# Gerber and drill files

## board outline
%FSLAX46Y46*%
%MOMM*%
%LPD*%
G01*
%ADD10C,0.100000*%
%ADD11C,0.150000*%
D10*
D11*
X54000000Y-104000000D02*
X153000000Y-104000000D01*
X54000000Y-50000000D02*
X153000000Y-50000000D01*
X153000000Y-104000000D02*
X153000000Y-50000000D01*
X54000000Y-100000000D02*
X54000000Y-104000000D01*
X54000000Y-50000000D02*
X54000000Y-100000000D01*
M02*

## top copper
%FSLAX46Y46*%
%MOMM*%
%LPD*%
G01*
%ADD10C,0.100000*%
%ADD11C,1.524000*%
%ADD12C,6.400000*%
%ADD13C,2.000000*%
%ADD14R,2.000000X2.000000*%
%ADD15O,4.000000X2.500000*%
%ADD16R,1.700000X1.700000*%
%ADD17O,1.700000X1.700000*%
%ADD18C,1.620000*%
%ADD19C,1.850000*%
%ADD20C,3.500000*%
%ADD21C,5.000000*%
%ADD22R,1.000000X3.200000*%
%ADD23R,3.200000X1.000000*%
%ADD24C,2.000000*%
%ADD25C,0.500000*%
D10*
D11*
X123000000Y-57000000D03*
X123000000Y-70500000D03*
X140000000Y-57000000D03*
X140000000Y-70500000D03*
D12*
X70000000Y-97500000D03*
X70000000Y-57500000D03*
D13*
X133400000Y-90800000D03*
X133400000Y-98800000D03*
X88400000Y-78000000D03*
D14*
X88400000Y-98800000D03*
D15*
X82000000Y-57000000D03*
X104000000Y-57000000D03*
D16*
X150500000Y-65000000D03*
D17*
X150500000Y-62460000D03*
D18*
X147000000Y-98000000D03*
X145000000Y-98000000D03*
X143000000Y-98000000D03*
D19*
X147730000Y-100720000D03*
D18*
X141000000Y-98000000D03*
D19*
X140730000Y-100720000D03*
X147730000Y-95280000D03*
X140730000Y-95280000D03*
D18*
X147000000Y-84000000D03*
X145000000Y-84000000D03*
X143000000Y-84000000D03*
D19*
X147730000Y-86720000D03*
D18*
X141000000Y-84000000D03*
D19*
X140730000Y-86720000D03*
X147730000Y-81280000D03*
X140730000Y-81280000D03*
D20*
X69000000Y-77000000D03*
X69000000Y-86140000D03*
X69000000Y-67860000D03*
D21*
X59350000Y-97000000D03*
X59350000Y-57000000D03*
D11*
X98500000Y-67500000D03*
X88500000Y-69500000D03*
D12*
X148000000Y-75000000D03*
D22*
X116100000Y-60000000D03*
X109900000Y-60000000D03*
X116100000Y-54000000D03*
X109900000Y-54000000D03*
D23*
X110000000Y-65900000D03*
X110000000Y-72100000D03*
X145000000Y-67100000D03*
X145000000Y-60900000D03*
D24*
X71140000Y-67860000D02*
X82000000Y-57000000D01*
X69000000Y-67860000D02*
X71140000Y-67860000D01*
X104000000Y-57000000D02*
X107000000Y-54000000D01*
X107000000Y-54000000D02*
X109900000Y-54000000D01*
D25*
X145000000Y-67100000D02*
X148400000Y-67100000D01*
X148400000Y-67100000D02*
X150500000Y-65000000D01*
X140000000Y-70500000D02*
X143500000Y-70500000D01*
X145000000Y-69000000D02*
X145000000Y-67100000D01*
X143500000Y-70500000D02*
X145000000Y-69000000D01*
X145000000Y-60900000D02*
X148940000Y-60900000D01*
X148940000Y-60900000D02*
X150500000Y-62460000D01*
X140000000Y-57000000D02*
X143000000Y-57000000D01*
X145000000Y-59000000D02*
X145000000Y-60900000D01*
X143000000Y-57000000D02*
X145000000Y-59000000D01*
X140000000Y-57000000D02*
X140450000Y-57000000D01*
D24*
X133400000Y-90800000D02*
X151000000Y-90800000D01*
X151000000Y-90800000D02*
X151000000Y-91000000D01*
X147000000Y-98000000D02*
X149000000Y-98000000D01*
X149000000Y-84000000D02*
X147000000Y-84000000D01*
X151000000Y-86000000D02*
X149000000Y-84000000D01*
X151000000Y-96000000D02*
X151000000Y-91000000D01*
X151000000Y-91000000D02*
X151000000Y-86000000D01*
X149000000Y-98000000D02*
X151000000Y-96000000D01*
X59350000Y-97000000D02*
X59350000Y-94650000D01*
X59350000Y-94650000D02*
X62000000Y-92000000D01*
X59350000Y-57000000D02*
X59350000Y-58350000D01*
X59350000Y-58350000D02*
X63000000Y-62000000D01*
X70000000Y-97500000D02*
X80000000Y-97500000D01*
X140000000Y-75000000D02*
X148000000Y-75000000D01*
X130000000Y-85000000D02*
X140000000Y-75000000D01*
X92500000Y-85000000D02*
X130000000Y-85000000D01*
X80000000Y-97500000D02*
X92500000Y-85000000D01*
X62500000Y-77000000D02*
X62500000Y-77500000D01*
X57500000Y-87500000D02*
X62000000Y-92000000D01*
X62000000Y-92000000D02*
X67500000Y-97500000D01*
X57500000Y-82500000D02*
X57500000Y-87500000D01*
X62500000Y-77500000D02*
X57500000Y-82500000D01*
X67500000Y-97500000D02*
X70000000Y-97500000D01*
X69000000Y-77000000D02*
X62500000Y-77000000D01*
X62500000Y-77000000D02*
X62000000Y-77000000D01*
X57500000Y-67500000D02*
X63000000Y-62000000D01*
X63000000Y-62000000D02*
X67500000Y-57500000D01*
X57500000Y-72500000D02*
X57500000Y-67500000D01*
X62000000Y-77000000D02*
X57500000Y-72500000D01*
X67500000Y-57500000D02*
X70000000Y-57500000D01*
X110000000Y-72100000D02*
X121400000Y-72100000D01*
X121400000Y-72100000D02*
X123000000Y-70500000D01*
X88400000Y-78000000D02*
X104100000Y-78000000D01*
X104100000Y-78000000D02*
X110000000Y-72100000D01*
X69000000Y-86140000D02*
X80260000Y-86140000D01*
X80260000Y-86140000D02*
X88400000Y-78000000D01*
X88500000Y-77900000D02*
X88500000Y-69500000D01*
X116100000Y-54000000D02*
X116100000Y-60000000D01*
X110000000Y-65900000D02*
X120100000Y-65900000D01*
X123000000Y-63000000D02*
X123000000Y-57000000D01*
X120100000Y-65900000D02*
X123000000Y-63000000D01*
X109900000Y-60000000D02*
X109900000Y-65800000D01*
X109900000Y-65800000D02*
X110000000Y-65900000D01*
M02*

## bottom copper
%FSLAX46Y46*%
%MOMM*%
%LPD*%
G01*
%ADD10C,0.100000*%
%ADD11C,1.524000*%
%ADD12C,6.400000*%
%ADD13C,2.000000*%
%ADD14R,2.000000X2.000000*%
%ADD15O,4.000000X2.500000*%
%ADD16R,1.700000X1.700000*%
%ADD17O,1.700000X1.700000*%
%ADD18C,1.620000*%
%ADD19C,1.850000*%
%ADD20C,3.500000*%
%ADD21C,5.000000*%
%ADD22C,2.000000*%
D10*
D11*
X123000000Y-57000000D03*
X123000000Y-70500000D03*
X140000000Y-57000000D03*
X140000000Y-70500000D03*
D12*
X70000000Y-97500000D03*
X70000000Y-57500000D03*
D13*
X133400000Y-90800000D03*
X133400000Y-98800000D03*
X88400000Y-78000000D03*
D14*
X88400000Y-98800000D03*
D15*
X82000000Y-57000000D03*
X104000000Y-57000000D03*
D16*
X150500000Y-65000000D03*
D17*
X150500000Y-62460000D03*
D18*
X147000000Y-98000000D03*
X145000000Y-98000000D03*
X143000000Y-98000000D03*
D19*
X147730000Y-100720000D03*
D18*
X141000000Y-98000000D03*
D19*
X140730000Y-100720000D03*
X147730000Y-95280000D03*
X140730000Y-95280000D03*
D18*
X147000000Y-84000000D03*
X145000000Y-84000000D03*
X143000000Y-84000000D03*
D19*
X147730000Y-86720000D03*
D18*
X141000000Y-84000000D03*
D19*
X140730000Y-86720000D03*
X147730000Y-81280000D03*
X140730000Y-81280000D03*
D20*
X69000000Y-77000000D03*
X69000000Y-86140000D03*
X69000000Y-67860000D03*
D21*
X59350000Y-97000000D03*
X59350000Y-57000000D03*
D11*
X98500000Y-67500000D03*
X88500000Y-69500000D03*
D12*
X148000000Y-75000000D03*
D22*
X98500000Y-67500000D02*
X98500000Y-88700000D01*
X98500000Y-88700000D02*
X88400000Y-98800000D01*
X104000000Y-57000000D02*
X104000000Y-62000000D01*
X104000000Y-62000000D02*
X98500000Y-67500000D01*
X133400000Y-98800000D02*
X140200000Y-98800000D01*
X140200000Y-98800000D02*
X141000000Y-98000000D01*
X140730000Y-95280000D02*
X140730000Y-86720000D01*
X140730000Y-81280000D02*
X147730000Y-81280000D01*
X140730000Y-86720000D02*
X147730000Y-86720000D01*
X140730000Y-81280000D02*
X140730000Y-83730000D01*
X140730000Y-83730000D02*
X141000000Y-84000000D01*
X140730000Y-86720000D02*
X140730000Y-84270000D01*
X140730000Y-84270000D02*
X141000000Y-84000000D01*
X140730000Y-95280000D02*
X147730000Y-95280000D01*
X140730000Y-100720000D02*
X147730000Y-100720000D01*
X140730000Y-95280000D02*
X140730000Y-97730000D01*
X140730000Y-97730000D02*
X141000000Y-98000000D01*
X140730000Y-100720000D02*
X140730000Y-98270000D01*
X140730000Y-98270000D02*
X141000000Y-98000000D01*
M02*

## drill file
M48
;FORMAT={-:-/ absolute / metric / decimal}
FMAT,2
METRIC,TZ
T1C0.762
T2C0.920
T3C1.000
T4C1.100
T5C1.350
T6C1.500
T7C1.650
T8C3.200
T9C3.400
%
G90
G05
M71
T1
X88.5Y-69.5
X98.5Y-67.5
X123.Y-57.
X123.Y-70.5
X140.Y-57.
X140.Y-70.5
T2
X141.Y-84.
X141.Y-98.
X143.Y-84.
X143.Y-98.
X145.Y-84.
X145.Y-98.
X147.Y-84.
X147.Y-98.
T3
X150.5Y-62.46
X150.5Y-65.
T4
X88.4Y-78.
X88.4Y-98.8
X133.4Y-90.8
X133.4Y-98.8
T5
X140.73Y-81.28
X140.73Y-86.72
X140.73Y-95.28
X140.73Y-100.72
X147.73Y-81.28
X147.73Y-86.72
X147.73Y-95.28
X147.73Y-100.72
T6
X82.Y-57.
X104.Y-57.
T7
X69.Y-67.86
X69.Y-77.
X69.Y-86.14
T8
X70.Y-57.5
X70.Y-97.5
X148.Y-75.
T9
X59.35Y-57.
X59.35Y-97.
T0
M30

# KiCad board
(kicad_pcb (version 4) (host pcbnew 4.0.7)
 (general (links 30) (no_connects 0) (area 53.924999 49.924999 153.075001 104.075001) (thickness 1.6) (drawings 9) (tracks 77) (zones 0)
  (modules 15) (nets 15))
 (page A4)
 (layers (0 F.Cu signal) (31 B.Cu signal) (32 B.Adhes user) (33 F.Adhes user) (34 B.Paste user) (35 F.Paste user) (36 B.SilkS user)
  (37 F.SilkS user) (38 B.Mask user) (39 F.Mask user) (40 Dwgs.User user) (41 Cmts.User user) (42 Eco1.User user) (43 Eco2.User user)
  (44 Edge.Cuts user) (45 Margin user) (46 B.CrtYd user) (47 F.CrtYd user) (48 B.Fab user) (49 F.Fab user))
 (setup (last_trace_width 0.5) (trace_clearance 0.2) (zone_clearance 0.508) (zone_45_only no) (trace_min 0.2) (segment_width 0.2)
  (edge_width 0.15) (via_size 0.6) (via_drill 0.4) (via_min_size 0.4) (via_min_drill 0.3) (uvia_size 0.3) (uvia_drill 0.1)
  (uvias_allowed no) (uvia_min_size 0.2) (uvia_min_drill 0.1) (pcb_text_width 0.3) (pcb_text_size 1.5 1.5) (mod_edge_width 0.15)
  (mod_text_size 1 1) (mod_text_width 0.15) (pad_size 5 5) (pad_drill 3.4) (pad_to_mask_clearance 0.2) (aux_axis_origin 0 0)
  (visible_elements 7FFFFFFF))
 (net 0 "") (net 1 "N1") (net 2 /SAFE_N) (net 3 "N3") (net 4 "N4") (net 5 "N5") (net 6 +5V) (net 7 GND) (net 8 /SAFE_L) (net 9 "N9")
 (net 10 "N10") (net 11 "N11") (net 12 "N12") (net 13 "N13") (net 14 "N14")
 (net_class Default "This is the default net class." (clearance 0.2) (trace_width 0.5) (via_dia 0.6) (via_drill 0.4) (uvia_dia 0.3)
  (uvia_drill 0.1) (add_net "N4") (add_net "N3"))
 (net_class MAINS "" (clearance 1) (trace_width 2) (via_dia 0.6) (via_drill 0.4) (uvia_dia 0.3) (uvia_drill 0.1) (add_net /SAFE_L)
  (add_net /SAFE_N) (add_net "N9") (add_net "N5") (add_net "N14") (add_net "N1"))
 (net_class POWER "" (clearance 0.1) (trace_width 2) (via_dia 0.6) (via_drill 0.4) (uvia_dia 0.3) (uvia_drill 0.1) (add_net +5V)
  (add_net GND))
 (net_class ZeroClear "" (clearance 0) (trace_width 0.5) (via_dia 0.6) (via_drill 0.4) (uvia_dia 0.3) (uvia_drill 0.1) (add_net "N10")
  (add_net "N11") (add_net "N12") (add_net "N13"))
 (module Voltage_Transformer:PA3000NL (layer F.Cu) (at 123 57)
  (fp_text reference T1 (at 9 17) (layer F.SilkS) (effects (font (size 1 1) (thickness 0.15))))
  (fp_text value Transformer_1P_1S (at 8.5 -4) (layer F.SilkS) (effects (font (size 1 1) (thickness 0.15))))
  (pad 1 thru_hole circle (at 0 0) (size 1.524 1.524) (drill 0.762) (layers *.Cu *.Mask) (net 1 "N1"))
  (pad 2 thru_hole circle (at 0 13.5) (size 1.524 1.524) (drill 0.762) (layers *.Cu *.Mask) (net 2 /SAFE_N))
  (pad 3 thru_hole circle (at 17 0) (size 1.524 1.524) (drill 0.762) (layers *.Cu *.Mask) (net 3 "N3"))
  (pad 4 thru_hole circle (at 17 13.5) (size 1.524 1.524) (drill 0.762) (layers *.Cu *.Mask) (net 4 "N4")))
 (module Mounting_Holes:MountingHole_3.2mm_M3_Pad (layer F.Cu) (at 70 97.5)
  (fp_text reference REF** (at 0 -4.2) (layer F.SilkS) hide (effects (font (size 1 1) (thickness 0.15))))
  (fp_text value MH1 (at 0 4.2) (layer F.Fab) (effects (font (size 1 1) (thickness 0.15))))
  (pad 1 thru_hole circle (at 0 0) (size 6.4 6.4) (drill 3.2) (layers *.Cu *.Mask) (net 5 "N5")))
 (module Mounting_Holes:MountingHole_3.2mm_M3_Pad (layer F.Cu) (at 70 57.5)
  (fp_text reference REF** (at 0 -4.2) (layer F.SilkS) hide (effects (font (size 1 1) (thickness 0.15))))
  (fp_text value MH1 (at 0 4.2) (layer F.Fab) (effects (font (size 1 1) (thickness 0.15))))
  (pad 1 thru_hole circle (at 0 0) (size 6.4 6.4) (drill 3.2) (layers *.Cu *.Mask) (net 5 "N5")))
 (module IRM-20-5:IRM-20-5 (layer F.Cu) (at 85 102)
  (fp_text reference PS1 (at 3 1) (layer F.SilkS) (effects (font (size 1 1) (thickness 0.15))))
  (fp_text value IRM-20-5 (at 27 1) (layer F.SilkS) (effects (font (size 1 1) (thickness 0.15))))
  (pad 4 thru_hole circle (at 48.4 -11.2 270) (size 2 2) (drill 1.1) (layers *.Cu *.Mask) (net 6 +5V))
  (pad 3 thru_hole circle (at 48.4 -3.2 270) (size 2 2) (drill 1.1) (layers *.Cu *.Mask) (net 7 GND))
  (pad 2 thru_hole circle (at 3.4 -24 270) (size 2 2) (drill 1.1) (layers *.Cu *.Mask) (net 2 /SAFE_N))
  (pad 1 thru_hole rect (at 3.4 -3.2 270) (size 2 2) (drill 1.1) (layers *.Cu *.Mask) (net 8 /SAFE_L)))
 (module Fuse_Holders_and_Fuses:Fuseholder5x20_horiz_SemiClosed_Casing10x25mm (layer F.Cu) (at 104 57 180)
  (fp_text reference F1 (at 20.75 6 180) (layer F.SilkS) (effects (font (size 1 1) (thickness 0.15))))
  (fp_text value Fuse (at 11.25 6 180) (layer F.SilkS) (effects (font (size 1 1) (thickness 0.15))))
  (pad 2 thru_hole oval (at 22 0 90) (size 2.5 4) (drill 1.5) (layers *.Cu *.Mask) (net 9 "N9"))
  (pad 1 thru_hole oval (at 0 0 90) (size 2.5 4) (drill 1.5) (layers *.Cu *.Mask) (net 8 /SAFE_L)))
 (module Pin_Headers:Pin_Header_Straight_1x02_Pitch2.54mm (layer F.Cu) (at 150.5 65 180)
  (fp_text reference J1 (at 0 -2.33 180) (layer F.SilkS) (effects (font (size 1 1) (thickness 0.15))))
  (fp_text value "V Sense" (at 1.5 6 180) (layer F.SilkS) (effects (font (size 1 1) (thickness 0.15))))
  (pad 1 thru_hole rect (at 0 0 180) (size 1.7 1.7) (drill 1) (layers *.Cu *.Mask) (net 4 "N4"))
  (pad 2 thru_hole oval (at 0 2.54 180) (size 1.7 1.7) (drill 1) (layers *.Cu *.Mask) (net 3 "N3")))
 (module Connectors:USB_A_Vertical (layer F.Cu) (at 147 98 270)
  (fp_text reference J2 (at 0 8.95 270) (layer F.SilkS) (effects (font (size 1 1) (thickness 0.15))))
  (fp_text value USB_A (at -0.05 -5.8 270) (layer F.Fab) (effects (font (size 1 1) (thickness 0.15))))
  (pad 1 thru_hole circle (at 0 0 270) (size 1.62 1.62) (drill 0.92) (layers *.Cu *.Mask) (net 6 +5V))
  (pad 2 thru_hole circle (at 0 2 270) (size 1.62 1.62) (drill 0.92) (layers *.Cu *.Mask) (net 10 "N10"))
  (pad 3 thru_hole circle (at 0 4 270) (size 1.62 1.62) (drill 0.92) (layers *.Cu *.Mask) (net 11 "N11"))
  (pad 5 thru_hole circle (at 2.72 -0.73 270) (size 1.85 1.85) (drill 1.35) (layers *.Cu *.Mask) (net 7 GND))
  (pad 4 thru_hole circle (at 0 6 270) (size 1.62 1.62) (drill 0.92) (layers *.Cu *.Mask) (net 7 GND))
  (pad 5 thru_hole circle (at 2.72 6.27 270) (size 1.85 1.85) (drill 1.35) (layers *.Cu *.Mask) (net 7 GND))
  (pad 5 thru_hole circle (at -2.72 -0.73 270) (size 1.85 1.85) (drill 1.35) (layers *.Cu *.Mask) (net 7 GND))
  (pad 5 thru_hole circle (at -2.72 6.27 270) (size 1.85 1.85) (drill 1.35) (layers *.Cu *.Mask) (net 7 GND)))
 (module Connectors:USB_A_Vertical (layer F.Cu) (at 147 84 270)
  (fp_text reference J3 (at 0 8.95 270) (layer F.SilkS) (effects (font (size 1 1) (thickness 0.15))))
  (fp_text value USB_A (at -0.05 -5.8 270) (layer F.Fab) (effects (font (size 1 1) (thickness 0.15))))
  (pad 1 thru_hole circle (at 0 0 270) (size 1.62 1.62) (drill 0.92) (layers *.Cu *.Mask) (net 6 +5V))
  (pad 2 thru_hole circle (at 0 2 270) (size 1.62 1.62) (drill 0.92) (layers *.Cu *.Mask) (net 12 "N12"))
  (pad 3 thru_hole circle (at 0 4 270) (size 1.62 1.62) (drill 0.92) (layers *.Cu *.Mask) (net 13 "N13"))
  (pad 5 thru_hole circle (at 2.72 -0.73 270) (size 1.85 1.85) (drill 1.35) (layers *.Cu *.Mask) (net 7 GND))
  (pad 4 thru_hole circle (at 0 6 270) (size 1.62 1.62) (drill 0.92) (layers *.Cu *.Mask) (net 7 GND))
  (pad 5 thru_hole circle (at 2.72 6.27 270) (size 1.85 1.85) (drill 1.35) (layers *.Cu *.Mask) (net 7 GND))
  (pad 5 thru_hole circle (at -2.72 -0.73 270) (size 1.85 1.85) (drill 1.35) (layers *.Cu *.Mask) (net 7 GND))
  (pad 5 thru_hole circle (at -2.72 6.27 270) (size 1.85 1.85) (drill 1.35) (layers *.Cu *.Mask) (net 7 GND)))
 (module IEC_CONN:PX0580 (layer F.Cu) (at 69 77 90)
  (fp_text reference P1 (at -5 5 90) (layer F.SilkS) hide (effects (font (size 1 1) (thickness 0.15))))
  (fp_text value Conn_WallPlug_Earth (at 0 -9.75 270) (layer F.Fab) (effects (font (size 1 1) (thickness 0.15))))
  (pad 3 thru_hole circle (at 0 0 90) (size 3.5 3.5) (drill 1.65) (layers *.Cu *.Mask) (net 5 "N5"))
  (pad 2 thru_hole circle (at -9.14 0 90) (size 3.5 3.5) (drill 1.65) (layers *.Cu *.Mask) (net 2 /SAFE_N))
  (pad 1 thru_hole circle (at 9.14 0 90) (size 3.5 3.5) (drill 1.65) (layers *.Cu *.Mask) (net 9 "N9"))
  (pad "" thru_hole circle (at -20 -9.65 90) (size 5 5) (drill 3.4) (layers *.Cu *.Mask))
  (pad "" thru_hole circle (at 20 -9.65 90) (size 5 5) (drill 3.4) (layers *.Cu *.Mask)))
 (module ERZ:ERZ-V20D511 (layer F.Cu) (at 104 65 180)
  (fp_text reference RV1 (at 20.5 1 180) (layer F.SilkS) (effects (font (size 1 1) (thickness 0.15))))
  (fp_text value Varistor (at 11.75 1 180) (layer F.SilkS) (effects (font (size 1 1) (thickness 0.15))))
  (pad 1 thru_hole circle (at 5.5 -2.5 180) (size 1.524 1.524) (drill 0.762) (layers *.Cu *.Mask) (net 8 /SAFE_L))
  (pad 2 thru_hole circle (at 15.5 -4.5 180) (size 1.524 1.524) (drill 0.762) (layers *.Cu *.Mask) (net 2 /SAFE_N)))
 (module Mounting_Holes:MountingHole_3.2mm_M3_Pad (layer F.Cu) (at 148 75)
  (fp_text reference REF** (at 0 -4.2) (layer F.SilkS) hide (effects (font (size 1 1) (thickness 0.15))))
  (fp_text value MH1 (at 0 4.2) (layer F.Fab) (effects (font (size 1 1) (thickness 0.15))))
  (pad 1 thru_hole circle (at 0 0) (size 6.4 6.4) (drill 3.2) (layers *.Cu *.Mask) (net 5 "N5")))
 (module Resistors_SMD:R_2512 (layer F.Cu) (at 113 60 180)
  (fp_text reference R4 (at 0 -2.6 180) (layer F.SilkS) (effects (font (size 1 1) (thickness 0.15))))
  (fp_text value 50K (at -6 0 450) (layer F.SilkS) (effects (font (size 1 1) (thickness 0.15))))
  (pad 1 smd rect (at -3.1 0 180) (size 1 3.2) (layers F.Cu F.Paste F.Mask) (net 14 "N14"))
  (pad 2 smd rect (at 3.1 0 180) (size 1 3.2) (layers F.Cu F.Paste F.Mask) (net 1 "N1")))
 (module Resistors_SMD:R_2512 (layer F.Cu) (at 113 54 180)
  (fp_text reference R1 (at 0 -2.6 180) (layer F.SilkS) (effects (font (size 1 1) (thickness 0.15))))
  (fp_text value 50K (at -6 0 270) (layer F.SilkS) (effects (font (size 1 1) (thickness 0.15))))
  (pad 1 smd rect (at -3.1 0 180) (size 1 3.2) (layers F.Cu F.Paste F.Mask) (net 14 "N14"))
  (pad 2 smd rect (at 3.1 0 180) (size 1 3.2) (layers F.Cu F.Paste F.Mask) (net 8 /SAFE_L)))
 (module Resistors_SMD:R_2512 (layer F.Cu) (at 110 69 270)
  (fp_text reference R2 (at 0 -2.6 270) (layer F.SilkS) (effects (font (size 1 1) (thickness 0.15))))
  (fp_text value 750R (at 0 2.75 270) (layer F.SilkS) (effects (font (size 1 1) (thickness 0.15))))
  (pad 1 smd rect (at -3.1 0 270) (size 1 3.2) (layers F.Cu F.Paste F.Mask) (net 1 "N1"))
  (pad 2 smd rect (at 3.1 0 270) (size 1 3.2) (layers F.Cu F.Paste F.Mask) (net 2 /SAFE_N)))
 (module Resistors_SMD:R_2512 (layer F.Cu) (at 145 64 90)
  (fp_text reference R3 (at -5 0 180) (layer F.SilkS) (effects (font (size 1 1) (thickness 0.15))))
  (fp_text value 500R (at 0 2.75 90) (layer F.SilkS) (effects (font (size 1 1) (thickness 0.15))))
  (pad 1 smd rect (at -3.1 0 90) (size 1 3.2) (layers F.Cu F.Paste F.Mask) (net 4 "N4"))
  (pad 2 smd rect (at 3.1 0 90) (size 1 3.2) (layers F.Cu F.Paste F.Mask) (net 3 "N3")))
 (gr_line (start 54 104) (end 153 104) (angle 90) (layer Edge.Cuts) (width 0.15))
 (gr_line (start 54 50) (end 153 50) (angle 90) (layer Edge.Cuts) (width 0.15))
 (gr_line (start 153 104) (end 153 50) (angle 90) (layer Edge.Cuts) (width 0.15))
 (gr_line (start 54 100) (end 54 104) (angle 90) (layer Edge.Cuts) (width 0.15))
 (gr_line (start 54 50) (end 54 100) (angle 90) (layer Edge.Cuts) (width 0.15))
 (segment (start 71.14 67.86) (end 82 57) (width 2) (layer F.Cu) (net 9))
 (segment (start 69 67.86) (end 71.14 67.86) (width 2) (layer F.Cu) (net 9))
 (segment (start 104 57) (end 107 54) (width 2) (layer F.Cu) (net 8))
 (segment (start 107 54) (end 109.9 54) (width 2) (layer F.Cu) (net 8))
 (segment (start 98.5 67.5) (end 98.5 88.7) (width 2) (layer B.Cu) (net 8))
 (segment (start 98.5 88.7) (end 88.4 98.8) (width 2) (layer B.Cu) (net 8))
 (segment (start 104 57) (end 104 62) (width 2) (layer B.Cu) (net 8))
 (segment (start 104 62) (end 98.5 67.5) (width 2) (layer B.Cu) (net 8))
 (segment (start 145 67.1) (end 148.4 67.1) (width 0.5) (layer F.Cu) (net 4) (status 400000))
 (segment (start 148.4 67.1) (end 150.5 65) (width 0.5) (layer F.Cu) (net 4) (status 800000))
 (segment (start 140 70.5) (end 143.5 70.5) (width 0.5) (layer F.Cu) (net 4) (status 400000))
 (segment (start 145 69) (end 145 67.1) (width 0.5) (layer F.Cu) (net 4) (status 800000))
 (segment (start 143.5 70.5) (end 145 69) (width 0.5) (layer F.Cu) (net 4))
 (segment (start 145 60.9) (end 148.94 60.9) (width 0.5) (layer F.Cu) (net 3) (status 400000))
 (segment (start 148.94 60.9) (end 150.5 62.46) (width 0.5) (layer F.Cu) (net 3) (status 800000))
 (segment (start 140 57) (end 143 57) (width 0.5) (layer F.Cu) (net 3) (status 400000))
 (segment (start 145 59) (end 145 60.9) (width 0.5) (layer F.Cu) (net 3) (status 800000))
 (segment (start 143 57) (end 145 59) (width 0.5) (layer F.Cu) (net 3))
 (segment (start 140 57) (end 140.45 57) (width 0.5) (layer F.Cu) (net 3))
 (segment (start 133.4 90.8) (end 151 90.8) (width 2) (layer F.Cu) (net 6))
 (segment (start 151 90.8) (end 151 91) (width 2) (layer F.Cu) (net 6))
 (segment (start 147 98) (end 149 98) (width 2) (layer F.Cu) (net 6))
 (segment (start 149 84) (end 147 84) (width 2) (layer F.Cu) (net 6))
 (segment (start 151 86) (end 149 84) (width 2) (layer F.Cu) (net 6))
 (segment (start 151 96) (end 151 91) (width 2) (layer F.Cu) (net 6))
 (segment (start 151 91) (end 151 86) (width 2) (layer F.Cu) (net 6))
 (segment (start 149 98) (end 151 96) (width 2) (layer F.Cu) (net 6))
 (segment (start 133.4 98.8) (end 140.2 98.8) (width 2) (layer B.Cu) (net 7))
 (segment (start 140.2 98.8) (end 141 98) (width 2) (layer B.Cu) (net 7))
 (segment (start 140.73 95.28) (end 140.73 86.72) (width 2) (layer B.Cu) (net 7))
 (segment (start 140.73 81.28) (end 147.73 81.28) (width 2) (layer B.Cu) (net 7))
 (segment (start 140.73 86.72) (end 147.73 86.72) (width 2) (layer B.Cu) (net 7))
 (segment (start 140.73 81.28) (end 140.73 83.73) (width 2) (layer B.Cu) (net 7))
 (segment (start 140.73 83.73) (end 141 84) (width 2) (layer B.Cu) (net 7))
 (segment (start 140.73 86.72) (end 140.73 84.27) (width 2) (layer B.Cu) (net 7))
 (segment (start 140.73 84.27) (end 141 84) (width 2) (layer B.Cu) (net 7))
 (segment (start 140.73 95.28) (end 147.73 95.28) (width 2) (layer B.Cu) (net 7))
 (segment (start 140.73 100.72) (end 147.73 100.72) (width 2) (layer B.Cu) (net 7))
 (segment (start 140.73 95.28) (end 140.73 97.73) (width 2) (layer B.Cu) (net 7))
 (segment (start 140.73 97.73) (end 141 98) (width 2) (layer B.Cu) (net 7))
 (segment (start 140.73 100.72) (end 140.73 98.27) (width 2) (layer B.Cu) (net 7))
 (segment (start 140.73 98.27) (end 141 98) (width 2) (layer B.Cu) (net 7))
 (segment (start 59.35 97) (end 59.35 94.65) (width 2) (layer F.Cu) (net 5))
 (segment (start 59.35 94.65) (end 62 92) (width 2) (layer F.Cu) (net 5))
 (segment (start 59.35 57) (end 59.35 58.35) (width 2) (layer F.Cu) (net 5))
 (segment (start 59.35 58.35) (end 63 62) (width 2) (layer F.Cu) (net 5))
 (segment (start 70 97.5) (end 80 97.5) (width 2) (layer F.Cu) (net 5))
 (segment (start 140 75) (end 148 75) (width 2) (layer F.Cu) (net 5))
 (segment (start 130 85) (end 140 75) (width 2) (layer F.Cu) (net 5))
 (segment (start 92.5 85) (end 130 85) (width 2) (layer F.Cu) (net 5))
 (segment (start 80 97.5) (end 92.5 85) (width 2) (layer F.Cu) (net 5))
 (segment (start 62.5 77) (end 62.5 77.5) (width 2) (layer F.Cu) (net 5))
 (segment (start 57.5 87.5) (end 62 92) (width 2) (layer F.Cu) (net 5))
 (segment (start 62 92) (end 67.5 97.5) (width 2) (layer F.Cu) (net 5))
 (segment (start 57.5 82.5) (end 57.5 87.5) (width 2) (layer F.Cu) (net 5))
 (segment (start 62.5 77.5) (end 57.5 82.5) (width 2) (layer F.Cu) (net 5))
 (segment (start 67.5 97.5) (end 70 97.5) (width 2) (layer F.Cu) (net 5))
 (segment (start 69 77) (end 62.5 77) (width 2) (layer F.Cu) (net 5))
 (segment (start 62.5 77) (end 62 77) (width 2) (layer F.Cu) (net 5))
 (segment (start 57.5 67.5) (end 63 62) (width 2) (layer F.Cu) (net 5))
 (segment (start 63 62) (end 67.5 57.5) (width 2) (layer F.Cu) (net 5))
 (segment (start 57.5 72.5) (end 57.5 67.5) (width 2) (layer F.Cu) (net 5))
 (segment (start 62 77) (end 57.5 72.5) (width 2) (layer F.Cu) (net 5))
 (segment (start 67.5 57.5) (end 70 57.5) (width 2) (layer F.Cu) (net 5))
 (segment (start 110 72.1) (end 121.4 72.1) (width 2) (layer F.Cu) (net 2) (status 400000))
 (segment (start 121.4 72.1) (end 123 70.5) (width 2) (layer F.Cu) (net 2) (status 800000))
 (segment (start 88.4 78) (end 104.1 78) (width 2) (layer F.Cu) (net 2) (status 400000))
 (segment (start 104.1 78) (end 110 72.1) (width 2) (layer F.Cu) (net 2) (status 800000))
 (segment (start 69 86.14) (end 80.26 86.14) (width 2) (layer F.Cu) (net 2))
 (segment (start 80.26 86.14) (end 88.4 78) (width 2) (layer F.Cu) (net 2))
 (segment (start 88.5 77.9) (end 88.5 69.5) (width 2) (layer F.Cu) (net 2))
 (segment (start 116.1 54) (end 116.1 60) (width 2) (layer F.Cu) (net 14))
 (segment (start 110 65.9) (end 120.1 65.9) (width 2) (layer F.Cu) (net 1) (status 400000))
 (segment (start 123 63) (end 123 57) (width 2) (layer F.Cu) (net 1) (status 800000))
 (segment (start 120.1 65.9) (end 123 63) (width 2) (layer F.Cu) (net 1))
 (segment (start 109.9 60) (end 109.9 65.8) (width 2) (layer F.Cu) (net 1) (status C00000))
 (segment (start 109.9 65.8) (end 110 65.9) (width 2) (layer F.Cu) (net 1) (status C00000)))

